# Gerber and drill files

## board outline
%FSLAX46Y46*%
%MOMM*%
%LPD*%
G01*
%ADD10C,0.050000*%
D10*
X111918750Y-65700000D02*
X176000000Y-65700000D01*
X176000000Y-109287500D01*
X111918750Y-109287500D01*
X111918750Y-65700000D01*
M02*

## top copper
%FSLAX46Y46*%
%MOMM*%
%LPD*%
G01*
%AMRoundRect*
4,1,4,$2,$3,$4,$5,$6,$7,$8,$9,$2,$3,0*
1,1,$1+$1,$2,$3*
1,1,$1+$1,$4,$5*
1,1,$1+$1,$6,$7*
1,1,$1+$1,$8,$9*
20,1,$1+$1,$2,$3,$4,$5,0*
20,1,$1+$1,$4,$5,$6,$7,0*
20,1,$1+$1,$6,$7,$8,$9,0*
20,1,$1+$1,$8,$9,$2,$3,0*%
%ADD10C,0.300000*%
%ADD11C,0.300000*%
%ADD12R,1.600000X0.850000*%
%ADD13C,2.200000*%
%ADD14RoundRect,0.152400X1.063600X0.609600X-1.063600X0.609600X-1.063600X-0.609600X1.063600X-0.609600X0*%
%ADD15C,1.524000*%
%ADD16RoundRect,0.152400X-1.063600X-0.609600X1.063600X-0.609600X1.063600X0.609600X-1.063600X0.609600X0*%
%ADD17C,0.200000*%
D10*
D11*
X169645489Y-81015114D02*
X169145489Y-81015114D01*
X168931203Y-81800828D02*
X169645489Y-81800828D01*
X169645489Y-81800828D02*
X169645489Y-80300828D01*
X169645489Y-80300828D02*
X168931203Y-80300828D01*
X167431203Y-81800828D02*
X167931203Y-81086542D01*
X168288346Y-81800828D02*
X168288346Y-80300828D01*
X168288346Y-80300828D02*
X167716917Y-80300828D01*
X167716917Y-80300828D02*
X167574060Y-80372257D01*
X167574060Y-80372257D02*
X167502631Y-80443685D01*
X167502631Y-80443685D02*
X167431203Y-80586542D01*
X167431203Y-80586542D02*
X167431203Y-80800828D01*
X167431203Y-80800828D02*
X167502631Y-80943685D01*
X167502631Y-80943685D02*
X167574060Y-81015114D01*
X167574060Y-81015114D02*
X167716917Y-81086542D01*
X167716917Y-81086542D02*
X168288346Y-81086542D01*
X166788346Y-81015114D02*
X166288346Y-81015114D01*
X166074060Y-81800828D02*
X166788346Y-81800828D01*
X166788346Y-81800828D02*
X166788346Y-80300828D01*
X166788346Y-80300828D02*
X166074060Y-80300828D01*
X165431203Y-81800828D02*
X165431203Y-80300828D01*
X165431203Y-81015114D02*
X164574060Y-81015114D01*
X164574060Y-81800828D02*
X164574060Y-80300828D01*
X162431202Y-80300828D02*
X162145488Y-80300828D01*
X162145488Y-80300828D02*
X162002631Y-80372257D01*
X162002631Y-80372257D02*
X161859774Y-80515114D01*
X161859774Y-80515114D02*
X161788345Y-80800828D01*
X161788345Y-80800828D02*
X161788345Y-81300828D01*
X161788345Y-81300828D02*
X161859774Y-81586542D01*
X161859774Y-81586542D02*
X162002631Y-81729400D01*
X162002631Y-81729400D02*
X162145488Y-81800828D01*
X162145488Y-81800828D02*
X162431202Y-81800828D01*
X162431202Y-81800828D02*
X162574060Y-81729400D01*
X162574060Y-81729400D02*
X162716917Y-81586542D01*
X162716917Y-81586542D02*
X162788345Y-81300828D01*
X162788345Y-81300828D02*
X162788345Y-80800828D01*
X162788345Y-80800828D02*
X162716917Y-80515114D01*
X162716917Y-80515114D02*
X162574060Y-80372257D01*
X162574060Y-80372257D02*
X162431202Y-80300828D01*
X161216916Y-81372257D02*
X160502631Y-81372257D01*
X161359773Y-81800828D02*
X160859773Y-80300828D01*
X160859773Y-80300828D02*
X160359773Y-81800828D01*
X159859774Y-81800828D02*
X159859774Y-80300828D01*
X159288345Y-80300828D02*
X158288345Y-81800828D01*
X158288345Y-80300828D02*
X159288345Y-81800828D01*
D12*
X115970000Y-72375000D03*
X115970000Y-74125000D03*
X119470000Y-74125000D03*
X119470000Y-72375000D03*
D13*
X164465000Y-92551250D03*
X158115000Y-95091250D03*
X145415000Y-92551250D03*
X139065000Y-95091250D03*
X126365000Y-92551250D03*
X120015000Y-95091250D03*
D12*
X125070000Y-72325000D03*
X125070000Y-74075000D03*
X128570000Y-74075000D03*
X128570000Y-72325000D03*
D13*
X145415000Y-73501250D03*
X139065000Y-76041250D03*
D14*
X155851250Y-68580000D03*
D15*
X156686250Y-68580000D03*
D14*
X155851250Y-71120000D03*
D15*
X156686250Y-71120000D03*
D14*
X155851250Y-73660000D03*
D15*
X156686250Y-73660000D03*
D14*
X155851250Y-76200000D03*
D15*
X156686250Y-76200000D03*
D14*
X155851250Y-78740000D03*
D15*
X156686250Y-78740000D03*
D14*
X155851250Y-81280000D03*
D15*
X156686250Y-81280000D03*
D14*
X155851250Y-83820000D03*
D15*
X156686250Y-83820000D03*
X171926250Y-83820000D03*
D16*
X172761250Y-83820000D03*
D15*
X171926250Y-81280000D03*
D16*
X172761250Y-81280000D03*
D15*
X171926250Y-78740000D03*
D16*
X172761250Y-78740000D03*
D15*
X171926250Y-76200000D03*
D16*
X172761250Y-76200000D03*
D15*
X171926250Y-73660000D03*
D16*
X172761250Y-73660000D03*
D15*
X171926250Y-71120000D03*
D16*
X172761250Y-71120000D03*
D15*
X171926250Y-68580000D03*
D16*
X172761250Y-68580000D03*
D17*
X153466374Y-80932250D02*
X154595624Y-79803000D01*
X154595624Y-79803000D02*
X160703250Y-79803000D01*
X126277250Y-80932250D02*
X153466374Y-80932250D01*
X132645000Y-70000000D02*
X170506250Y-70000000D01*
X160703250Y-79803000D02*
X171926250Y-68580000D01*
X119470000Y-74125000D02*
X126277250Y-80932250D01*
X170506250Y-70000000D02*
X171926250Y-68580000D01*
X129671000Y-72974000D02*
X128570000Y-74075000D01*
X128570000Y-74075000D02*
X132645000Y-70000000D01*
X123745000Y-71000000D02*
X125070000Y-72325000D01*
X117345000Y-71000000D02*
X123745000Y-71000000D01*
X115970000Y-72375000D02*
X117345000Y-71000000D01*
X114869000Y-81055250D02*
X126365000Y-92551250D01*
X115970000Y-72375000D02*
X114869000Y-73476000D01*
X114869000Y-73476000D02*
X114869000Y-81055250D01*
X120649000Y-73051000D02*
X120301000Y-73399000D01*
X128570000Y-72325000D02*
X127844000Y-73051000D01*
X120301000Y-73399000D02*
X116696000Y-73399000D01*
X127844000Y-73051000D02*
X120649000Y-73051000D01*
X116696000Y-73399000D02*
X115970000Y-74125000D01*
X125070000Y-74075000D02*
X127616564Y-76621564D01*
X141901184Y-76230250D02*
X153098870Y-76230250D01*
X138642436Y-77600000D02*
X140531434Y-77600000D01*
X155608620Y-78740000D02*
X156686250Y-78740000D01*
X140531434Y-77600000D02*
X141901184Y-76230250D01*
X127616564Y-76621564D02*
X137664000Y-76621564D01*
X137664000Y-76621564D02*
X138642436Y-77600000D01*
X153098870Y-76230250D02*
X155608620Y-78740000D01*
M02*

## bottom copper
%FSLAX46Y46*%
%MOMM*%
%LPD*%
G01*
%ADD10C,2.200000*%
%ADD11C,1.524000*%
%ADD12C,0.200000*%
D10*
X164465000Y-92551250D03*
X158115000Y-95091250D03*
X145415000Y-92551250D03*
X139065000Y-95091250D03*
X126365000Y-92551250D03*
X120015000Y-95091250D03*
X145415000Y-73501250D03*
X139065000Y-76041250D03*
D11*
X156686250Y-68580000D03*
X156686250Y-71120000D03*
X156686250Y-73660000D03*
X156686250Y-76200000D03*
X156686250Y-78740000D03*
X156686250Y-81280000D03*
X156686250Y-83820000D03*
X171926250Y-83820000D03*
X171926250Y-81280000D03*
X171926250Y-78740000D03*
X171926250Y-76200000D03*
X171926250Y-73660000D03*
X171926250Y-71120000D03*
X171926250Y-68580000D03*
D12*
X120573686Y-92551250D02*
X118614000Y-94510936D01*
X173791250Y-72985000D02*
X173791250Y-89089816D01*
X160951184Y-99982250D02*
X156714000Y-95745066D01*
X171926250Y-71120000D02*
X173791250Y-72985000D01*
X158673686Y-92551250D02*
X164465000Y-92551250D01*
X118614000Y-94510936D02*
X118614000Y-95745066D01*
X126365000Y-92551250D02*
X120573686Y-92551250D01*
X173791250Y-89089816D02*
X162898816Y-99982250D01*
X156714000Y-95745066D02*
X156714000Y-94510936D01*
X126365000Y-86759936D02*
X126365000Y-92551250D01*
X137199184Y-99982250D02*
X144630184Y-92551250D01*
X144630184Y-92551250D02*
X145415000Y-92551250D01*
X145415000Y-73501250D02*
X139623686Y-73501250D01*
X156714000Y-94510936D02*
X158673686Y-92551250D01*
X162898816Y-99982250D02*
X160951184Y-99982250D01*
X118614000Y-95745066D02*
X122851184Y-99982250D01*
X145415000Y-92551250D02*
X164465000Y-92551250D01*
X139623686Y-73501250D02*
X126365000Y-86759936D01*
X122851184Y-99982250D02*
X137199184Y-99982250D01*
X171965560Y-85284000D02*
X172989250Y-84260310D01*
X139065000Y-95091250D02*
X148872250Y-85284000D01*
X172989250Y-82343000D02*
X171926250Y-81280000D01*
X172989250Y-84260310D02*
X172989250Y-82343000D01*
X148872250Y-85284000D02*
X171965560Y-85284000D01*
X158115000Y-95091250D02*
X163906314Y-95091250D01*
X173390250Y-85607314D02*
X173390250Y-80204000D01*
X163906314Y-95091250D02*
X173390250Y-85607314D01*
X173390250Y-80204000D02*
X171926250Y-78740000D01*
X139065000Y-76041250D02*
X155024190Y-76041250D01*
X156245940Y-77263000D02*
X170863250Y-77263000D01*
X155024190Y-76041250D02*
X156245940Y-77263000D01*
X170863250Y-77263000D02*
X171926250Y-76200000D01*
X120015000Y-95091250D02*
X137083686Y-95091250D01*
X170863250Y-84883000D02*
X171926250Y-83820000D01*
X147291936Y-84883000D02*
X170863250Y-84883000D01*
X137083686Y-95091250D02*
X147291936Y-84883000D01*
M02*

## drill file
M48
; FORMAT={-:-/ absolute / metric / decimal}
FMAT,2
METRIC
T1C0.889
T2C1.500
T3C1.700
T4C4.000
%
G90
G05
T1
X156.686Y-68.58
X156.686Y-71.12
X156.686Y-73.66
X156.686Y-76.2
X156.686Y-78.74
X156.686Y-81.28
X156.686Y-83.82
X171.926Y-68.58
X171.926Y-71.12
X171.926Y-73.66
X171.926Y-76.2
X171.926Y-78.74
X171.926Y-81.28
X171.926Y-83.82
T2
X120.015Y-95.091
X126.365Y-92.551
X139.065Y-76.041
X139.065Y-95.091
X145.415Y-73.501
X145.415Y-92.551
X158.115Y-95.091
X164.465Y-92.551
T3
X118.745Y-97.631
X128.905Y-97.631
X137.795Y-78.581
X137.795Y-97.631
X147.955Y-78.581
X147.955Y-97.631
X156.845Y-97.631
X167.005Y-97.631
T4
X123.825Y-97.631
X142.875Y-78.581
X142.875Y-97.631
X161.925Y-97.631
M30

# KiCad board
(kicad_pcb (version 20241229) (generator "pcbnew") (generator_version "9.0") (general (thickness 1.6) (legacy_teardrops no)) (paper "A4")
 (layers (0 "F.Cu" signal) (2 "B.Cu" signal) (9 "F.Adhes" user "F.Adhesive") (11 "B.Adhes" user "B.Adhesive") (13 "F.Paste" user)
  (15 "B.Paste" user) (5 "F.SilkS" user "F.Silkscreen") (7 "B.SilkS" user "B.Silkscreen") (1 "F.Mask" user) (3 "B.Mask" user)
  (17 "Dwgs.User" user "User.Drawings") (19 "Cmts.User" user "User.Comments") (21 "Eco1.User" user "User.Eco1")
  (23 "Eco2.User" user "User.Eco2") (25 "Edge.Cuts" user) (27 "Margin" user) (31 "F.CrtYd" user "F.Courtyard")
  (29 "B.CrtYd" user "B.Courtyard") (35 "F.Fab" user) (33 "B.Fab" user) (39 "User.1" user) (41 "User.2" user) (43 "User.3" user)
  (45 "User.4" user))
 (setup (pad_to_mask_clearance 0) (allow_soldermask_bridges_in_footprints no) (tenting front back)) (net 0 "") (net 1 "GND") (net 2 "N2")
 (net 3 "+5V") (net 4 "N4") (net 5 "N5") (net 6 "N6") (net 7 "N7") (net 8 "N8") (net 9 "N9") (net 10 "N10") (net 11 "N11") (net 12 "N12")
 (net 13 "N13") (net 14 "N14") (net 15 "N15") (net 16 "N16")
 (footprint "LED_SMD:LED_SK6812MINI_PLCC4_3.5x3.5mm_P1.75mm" (layer "F.Cu") (at 117.72 73.25)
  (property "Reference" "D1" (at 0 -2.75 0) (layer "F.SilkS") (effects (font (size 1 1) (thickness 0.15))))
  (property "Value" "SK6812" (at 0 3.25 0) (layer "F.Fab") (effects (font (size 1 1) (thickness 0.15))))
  (pad "1" smd rect (at -1.75 -0.875) (size 1.6 0.85) (layers "F.Cu" "F.Mask" "F.Paste") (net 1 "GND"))
  (pad "2" smd rect (at -1.75 0.875) (size 1.6 0.85) (layers "F.Cu" "F.Mask" "F.Paste") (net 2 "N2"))
  (pad "3" smd rect (at 1.75 0.875) (size 1.6 0.85) (layers "F.Cu" "F.Mask" "F.Paste") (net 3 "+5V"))
  (pad "4" smd rect (at 1.75 -0.875) (size 1.6 0.85) (layers "F.Cu" "F.Mask" "F.Paste") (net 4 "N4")))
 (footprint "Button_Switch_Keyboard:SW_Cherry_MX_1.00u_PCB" (layer "F.Cu") (at 164.465 92.55125)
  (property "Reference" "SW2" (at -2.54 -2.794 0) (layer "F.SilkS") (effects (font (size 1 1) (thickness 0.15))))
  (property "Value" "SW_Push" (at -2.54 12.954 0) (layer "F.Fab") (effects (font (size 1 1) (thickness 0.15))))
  (pad "" np_thru_hole circle (at -7.62 5.08) (size 1.7 1.7) (drill 1.7) (layers "*.Cu" "*.Mask"))
  (pad "" np_thru_hole circle (at -2.54 5.08) (size 4 4) (drill 4) (layers "*.Cu" "*.Mask"))
  (pad "" np_thru_hole circle (at 2.54 5.08) (size 1.7 1.7) (drill 1.7) (layers "*.Cu" "*.Mask"))
  (pad "1" thru_hole circle (at 0 0) (size 2.2 2.2) (drill 1.5) (layers "*.Cu" "*.Mask") (remove_unused_layers no) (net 1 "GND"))
  (pad "2" thru_hole circle (at -6.35 2.54) (size 2.2 2.2) (drill 1.5) (layers "*.Cu" "*.Mask") (remove_unused_layers no) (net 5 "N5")))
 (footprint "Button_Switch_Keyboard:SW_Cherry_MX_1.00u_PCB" (layer "F.Cu") (at 145.415 92.55125)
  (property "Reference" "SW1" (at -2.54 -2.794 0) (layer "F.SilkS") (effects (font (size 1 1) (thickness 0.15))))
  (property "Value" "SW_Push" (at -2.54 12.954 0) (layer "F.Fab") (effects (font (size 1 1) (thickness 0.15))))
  (pad "" np_thru_hole circle (at -7.62 5.08) (size 1.7 1.7) (drill 1.7) (layers "*.Cu" "*.Mask"))
  (pad "" np_thru_hole circle (at -2.54 5.08) (size 4 4) (drill 4) (layers "*.Cu" "*.Mask"))
  (pad "" np_thru_hole circle (at 2.54 5.08) (size 1.7 1.7) (drill 1.7) (layers "*.Cu" "*.Mask"))
  (pad "1" thru_hole circle (at 0 0) (size 2.2 2.2) (drill 1.5) (layers "*.Cu" "*.Mask") (remove_unused_layers no) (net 1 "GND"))
  (pad "2" thru_hole circle (at -6.35 2.54) (size 2.2 2.2) (drill 1.5) (layers "*.Cu" "*.Mask") (remove_unused_layers no) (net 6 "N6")))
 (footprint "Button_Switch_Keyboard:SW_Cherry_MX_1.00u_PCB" (layer "F.Cu") (at 126.365 92.55125)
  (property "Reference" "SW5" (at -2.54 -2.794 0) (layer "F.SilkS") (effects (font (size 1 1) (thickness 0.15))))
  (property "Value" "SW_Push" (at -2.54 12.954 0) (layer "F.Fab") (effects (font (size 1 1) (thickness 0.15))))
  (pad "" np_thru_hole circle (at -7.62 5.08) (size 1.7 1.7) (drill 1.7) (layers "*.Cu" "*.Mask"))
  (pad "" np_thru_hole circle (at -2.54 5.08) (size 4 4) (drill 4) (layers "*.Cu" "*.Mask"))
  (pad "" np_thru_hole circle (at 2.54 5.08) (size 1.7 1.7) (drill 1.7) (layers "*.Cu" "*.Mask"))
  (pad "1" thru_hole circle (at 0 0) (size 2.2 2.2) (drill 1.5) (layers "*.Cu" "*.Mask") (remove_unused_layers no) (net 1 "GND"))
  (pad "2" thru_hole circle (at -6.35 2.54) (size 2.2 2.2) (drill 1.5) (layers "*.Cu" "*.Mask") (remove_unused_layers no) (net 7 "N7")))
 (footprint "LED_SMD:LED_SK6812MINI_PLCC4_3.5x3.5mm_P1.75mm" (layer "F.Cu") (at 126.82 73.2)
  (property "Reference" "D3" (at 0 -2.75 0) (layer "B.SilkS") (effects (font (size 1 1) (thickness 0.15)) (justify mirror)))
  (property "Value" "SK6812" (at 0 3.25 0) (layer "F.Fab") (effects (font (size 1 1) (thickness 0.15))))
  (pad "1" smd rect (at -1.75 -0.875) (size 1.6 0.85) (layers "F.Cu" "F.Mask" "F.Paste") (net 1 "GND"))
  (pad "2" smd rect (at -1.75 0.875) (size 1.6 0.85) (layers "F.Cu" "F.Mask" "F.Paste") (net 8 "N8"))
  (pad "3" smd rect (at 1.75 0.875) (size 1.6 0.85) (layers "F.Cu" "F.Mask" "F.Paste") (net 3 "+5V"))
  (pad "4" smd rect (at 1.75 -0.875) (size 1.6 0.85) (layers "F.Cu" "F.Mask" "F.Paste") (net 2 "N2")))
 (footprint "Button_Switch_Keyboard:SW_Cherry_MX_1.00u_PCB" (layer "F.Cu") (at 145.415 73.50125)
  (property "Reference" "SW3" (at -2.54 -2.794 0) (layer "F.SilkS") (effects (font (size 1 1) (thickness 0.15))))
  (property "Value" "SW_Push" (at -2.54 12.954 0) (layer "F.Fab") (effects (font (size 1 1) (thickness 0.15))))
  (pad "" np_thru_hole circle (at -7.62 5.08) (size 1.7 1.7) (drill 1.7) (layers "*.Cu" "*.Mask"))
  (pad "" np_thru_hole circle (at -2.54 5.08) (size 4 4) (drill 4) (layers "*.Cu" "*.Mask"))
  (pad "" np_thru_hole circle (at 2.54 5.08) (size 1.7 1.7) (drill 1.7) (layers "*.Cu" "*.Mask"))
  (pad "1" thru_hole circle (at 0 0) (size 2.2 2.2) (drill 1.5) (layers "*.Cu" "*.Mask") (remove_unused_layers no) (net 1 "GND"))
  (pad "2" thru_hole circle (at -6.35 2.54) (size 2.2 2.2) (drill 1.5) (layers "*.Cu" "*.Mask") (remove_unused_layers no) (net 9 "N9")))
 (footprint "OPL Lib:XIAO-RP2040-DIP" (layer "F.Cu") (at 164.30625 76.2)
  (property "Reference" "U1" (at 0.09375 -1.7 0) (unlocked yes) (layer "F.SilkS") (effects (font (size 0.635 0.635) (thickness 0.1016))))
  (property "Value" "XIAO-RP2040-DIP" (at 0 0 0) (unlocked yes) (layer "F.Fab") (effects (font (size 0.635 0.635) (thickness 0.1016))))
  (pad "1" smd roundrect (at -8.455 -7.62 180) (size 2.432 1.524) (layers "F.Cu" "F.Mask") (roundrect_rratio 0.1) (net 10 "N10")
   (thermal_bridge_angle 45))
  (pad "1" thru_hole circle (at -7.62 -7.62 180) (size 1.524 1.524) (drill 0.889) (layers "*.Cu" "*.Mask") (remove_unused_layers no)
   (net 10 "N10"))
  (pad "2" smd roundrect (at -8.455 -5.08 180) (size 2.432 1.524) (layers "F.Cu" "F.Mask") (roundrect_rratio 0.1) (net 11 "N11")
   (thermal_bridge_angle 45))
  (pad "2" thru_hole circle (at -7.62 -5.08 180) (size 1.524 1.524) (drill 0.889) (layers "*.Cu" "*.Mask") (remove_unused_layers no)
   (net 11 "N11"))
  (pad "3" smd roundrect (at -8.455 -2.54 180) (size 2.432 1.524) (layers "F.Cu" "F.Mask") (roundrect_rratio 0.1) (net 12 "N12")
   (thermal_bridge_angle 45))
  (pad "3" thru_hole circle (at -7.62 -2.54 180) (size 1.524 1.524) (drill 0.889) (layers "*.Cu" "*.Mask") (remove_unused_layers no)
   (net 12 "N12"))
  (pad "4" smd roundrect (at -8.455 0 180) (size 2.432 1.524) (layers "F.Cu" "F.Mask") (roundrect_rratio 0.1) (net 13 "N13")
   (thermal_bridge_angle 45))
  (pad "4" thru_hole circle (at -7.62 0 180) (size 1.524 1.524) (drill 0.889) (layers "*.Cu" "*.Mask") (remove_unused_layers no)
   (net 13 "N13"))
  (pad "5" smd roundrect (at -8.455 2.54 180) (size 2.432 1.524) (layers "F.Cu" "F.Mask") (roundrect_rratio 0.1) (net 8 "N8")
   (thermal_bridge_angle 45))
  (pad "5" thru_hole circle (at -7.62 2.54 180) (size 1.524 1.524) (drill 0.889) (layers "*.Cu" "*.Mask") (remove_unused_layers no)
   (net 8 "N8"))
  (pad "6" smd roundrect (at -8.455 5.08 180) (size 2.432 1.524) (layers "F.Cu" "F.Mask") (roundrect_rratio 0.1) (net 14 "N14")
   (thermal_bridge_angle 45))
  (pad "6" thru_hole circle (at -7.62 5.08 180) (size 1.524 1.524) (drill 0.889) (layers "*.Cu" "*.Mask") (remove_unused_layers no)
   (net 14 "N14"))
  (pad "7" smd roundrect (at -8.455 7.62 180) (size 2.432 1.524) (layers "F.Cu" "F.Mask") (roundrect_rratio 0.1) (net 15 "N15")
   (thermal_bridge_angle 45))
  (pad "7" thru_hole circle (at -7.62 7.62 180) (size 1.524 1.524) (drill 0.889) (layers "*.Cu" "*.Mask") (remove_unused_layers no)
   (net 15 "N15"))
  (pad "8" thru_hole circle (at 7.62 7.62) (size 1.524 1.524) (drill 0.889) (layers "*.Cu" "*.Mask") (remove_unused_layers no) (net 7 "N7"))
  (pad "8" smd roundrect (at 8.455 7.62) (size 2.432 1.524) (layers "F.Cu" "F.Mask") (roundrect_rratio 0.1) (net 7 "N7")
   (thermal_bridge_angle 45))
  (pad "9" thru_hole circle (at 7.62 5.08) (size 1.524 1.524) (drill 0.889) (layers "*.Cu" "*.Mask") (remove_unused_layers no) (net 6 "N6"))
  (pad "9" smd roundrect (at 8.455 5.08) (size 2.432 1.524) (layers "F.Cu" "F.Mask") (roundrect_rratio 0.1) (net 6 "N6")
   (thermal_bridge_angle 45))
  (pad "10" thru_hole circle (at 7.62 2.54) (size 1.524 1.524) (drill 0.889) (layers "*.Cu" "*.Mask") (remove_unused_layers no) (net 5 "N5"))
  (pad "10" smd roundrect (at 8.455 2.54) (size 2.432 1.524) (layers "F.Cu" "F.Mask") (roundrect_rratio 0.1) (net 5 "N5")
   (thermal_bridge_angle 45))
  (pad "11" thru_hole circle (at 7.62 0) (size 1.524 1.524) (drill 0.889) (layers "*.Cu" "*.Mask") (remove_unused_layers no) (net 9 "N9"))
  (pad "11" smd roundrect (at 8.455 0) (size 2.432 1.524) (layers "F.Cu" "F.Mask") (roundrect_rratio 0.1) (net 9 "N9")
   (thermal_bridge_angle 45))
  (pad "12" thru_hole circle (at 7.62 -2.54) (size 1.524 1.524) (drill 0.889) (layers "*.Cu" "*.Mask") (remove_unused_layers no)
   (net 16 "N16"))
  (pad "12" smd roundrect (at 8.455 -2.54) (size 2.432 1.524) (layers "F.Cu" "F.Mask") (roundrect_rratio 0.1) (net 16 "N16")
   (thermal_bridge_angle 45))
  (pad "13" thru_hole circle (at 7.62 -5.08) (size 1.524 1.524) (drill 0.889) (layers "*.Cu" "*.Mask") (remove_unused_layers no)
   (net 1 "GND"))
  (pad "13" smd roundrect (at 8.455 -5.08) (size 2.432 1.524) (layers "F.Cu" "F.Mask") (roundrect_rratio 0.1) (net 1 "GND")
   (thermal_bridge_angle 45))
  (pad "14" thru_hole circle (at 7.62 -7.62) (size 1.524 1.524) (drill 0.889) (layers "*.Cu" "*.Mask") (remove_unused_layers no)
   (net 3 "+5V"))
  (pad "14" smd roundrect (at 8.455 -7.62) (size 2.432 1.524) (layers "F.Cu" "F.Mask") (roundrect_rratio 0.1) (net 3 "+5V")
   (thermal_bridge_angle 45)))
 (gr_rect (start 111.91875 65.7) (end 176 109.2875) (stroke (width 0.05) (type default)) (fill no) (layer "Edge.Cuts"))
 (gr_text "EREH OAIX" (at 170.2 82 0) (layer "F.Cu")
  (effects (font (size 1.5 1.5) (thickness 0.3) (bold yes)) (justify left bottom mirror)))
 (segment (start 153.466374 80.93225) (end 154.595624 79.803) (width 0.2) (layer "F.Cu") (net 3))
 (segment (start 154.595624 79.803) (end 160.70325 79.803) (width 0.2) (layer "F.Cu") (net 3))
 (segment (start 126.27725 80.93225) (end 153.466374 80.93225) (width 0.2) (layer "F.Cu") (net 3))
 (segment (start 132.645 70) (end 170.50625 70) (width 0.2) (layer "F.Cu") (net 3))
 (segment (start 160.70325 79.803) (end 171.92625 68.58) (width 0.2) (layer "F.Cu") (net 3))
 (segment (start 119.47 74.125) (end 126.27725 80.93225) (width 0.2) (layer "F.Cu") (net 3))
 (segment (start 170.50625 70) (end 171.92625 68.58) (width 0.2) (layer "F.Cu") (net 3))
 (segment (start 129.671 72.974) (end 128.57 74.075) (width 0.2) (layer "F.Cu") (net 3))
 (segment (start 128.57 74.075) (end 132.645 70) (width 0.2) (layer "F.Cu") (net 3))
 (segment (start 123.745 71) (end 125.07 72.325) (width 0.2) (layer "F.Cu") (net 1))
 (segment (start 117.345 71) (end 123.745 71) (width 0.2) (layer "F.Cu") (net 1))
 (segment (start 115.97 72.375) (end 117.345 71) (width 0.2) (layer "F.Cu") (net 1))
 (segment (start 114.869 81.05525) (end 126.365 92.55125) (width 0.2) (layer "F.Cu") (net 1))
 (segment (start 115.97 72.375) (end 114.869 73.476) (width 0.2) (layer "F.Cu") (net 1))
 (segment (start 114.869 73.476) (end 114.869 81.05525) (width 0.2) (layer "F.Cu") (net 1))
 (segment (start 120.573686 92.55125) (end 118.614 94.510936) (width 0.2) (layer "B.Cu") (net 1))
 (segment (start 173.79125 72.985) (end 173.79125 89.089816) (width 0.2) (layer "B.Cu") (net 1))
 (segment (start 160.951184 99.98225) (end 156.714 95.745066) (width 0.2) (layer "B.Cu") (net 1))
 (segment (start 171.92625 71.12) (end 173.79125 72.985) (width 0.2) (layer "B.Cu") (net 1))
 (segment (start 158.673686 92.55125) (end 164.465 92.55125) (width 0.2) (layer "B.Cu") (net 1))
 (segment (start 118.614 94.510936) (end 118.614 95.745066) (width 0.2) (layer "B.Cu") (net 1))
 (segment (start 126.365 92.55125) (end 120.573686 92.55125) (width 0.2) (layer "B.Cu") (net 1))
 (segment (start 173.79125 89.089816) (end 162.898816 99.98225) (width 0.2) (layer "B.Cu") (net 1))
 (segment (start 156.714 95.745066) (end 156.714 94.510936) (width 0.2) (layer "B.Cu") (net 1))
 (segment (start 126.365 86.759936) (end 126.365 92.55125) (width 0.2) (layer "B.Cu") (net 1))
 (segment (start 137.199184 99.98225) (end 144.630184 92.55125) (width 0.2) (layer "B.Cu") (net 1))
 (segment (start 144.630184 92.55125) (end 145.415 92.55125) (width 0.2) (layer "B.Cu") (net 1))
 (segment (start 145.415 73.50125) (end 139.623686 73.50125) (width 0.2) (layer "B.Cu") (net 1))
 (segment (start 156.714 94.510936) (end 158.673686 92.55125) (width 0.2) (layer "B.Cu") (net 1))
 (segment (start 162.898816 99.98225) (end 160.951184 99.98225) (width 0.2) (layer "B.Cu") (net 1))
 (segment (start 118.614 95.745066) (end 122.851184 99.98225) (width 0.2) (layer "B.Cu") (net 1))
 (segment (start 145.415 92.55125) (end 164.465 92.55125) (width 0.2) (layer "B.Cu") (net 1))
 (segment (start 139.623686 73.50125) (end 126.365 86.759936) (width 0.2) (layer "B.Cu") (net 1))
 (segment (start 122.851184 99.98225) (end 137.199184 99.98225) (width 0.2) (layer "B.Cu") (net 1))
 (segment (start 120.649 73.051) (end 120.301 73.399) (width 0.2) (layer "F.Cu") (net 2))
 (segment (start 128.57 72.325) (end 127.844 73.051) (width 0.2) (layer "F.Cu") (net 2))
 (segment (start 120.301 73.399) (end 116.696 73.399) (width 0.2) (layer "F.Cu") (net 2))
 (segment (start 127.844 73.051) (end 120.649 73.051) (width 0.2) (layer "F.Cu") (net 2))
 (segment (start 116.696 73.399) (end 115.97 74.125) (width 0.2) (layer "F.Cu") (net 2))
 (segment (start 125.07 74.075) (end 127.616564 76.621564) (width 0.2) (layer "F.Cu") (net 8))
 (segment (start 141.901184 76.23025) (end 153.09887 76.23025) (width 0.2) (layer "F.Cu") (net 8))
 (segment (start 138.642436 77.6) (end 140.531434 77.6) (width 0.2) (layer "F.Cu") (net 8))
 (segment (start 155.60862 78.74) (end 156.68625 78.74) (width 0.2) (layer "F.Cu") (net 8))
 (segment (start 140.531434 77.6) (end 141.901184 76.23025) (width 0.2) (layer "F.Cu") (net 8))
 (segment (start 127.616564 76.621564) (end 137.664 76.621564) (width 0.2) (layer "F.Cu") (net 8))
 (segment (start 137.664 76.621564) (end 138.642436 77.6) (width 0.2) (layer "F.Cu") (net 8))
 (segment (start 153.09887 76.23025) (end 155.60862 78.74) (width 0.2) (layer "F.Cu") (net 8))
 (segment (start 171.96556 85.284) (end 172.98925 84.26031) (width 0.2) (layer "B.Cu") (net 6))
 (segment (start 139.065 95.09125) (end 148.87225 85.284) (width 0.2) (layer "B.Cu") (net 6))
 (segment (start 172.98925 82.343) (end 171.92625 81.28) (width 0.2) (layer "B.Cu") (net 6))
 (segment (start 172.98925 84.26031) (end 172.98925 82.343) (width 0.2) (layer "B.Cu") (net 6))
 (segment (start 148.87225 85.284) (end 171.96556 85.284) (width 0.2) (layer "B.Cu") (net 6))
 (segment (start 158.115 95.09125) (end 163.906314 95.09125) (width 0.2) (layer "B.Cu") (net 5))
 (segment (start 173.39025 85.607314) (end 173.39025 80.204) (width 0.2) (layer "B.Cu") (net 5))
 (segment (start 163.906314 95.09125) (end 173.39025 85.607314) (width 0.2) (layer "B.Cu") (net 5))
 (segment (start 173.39025 80.204) (end 171.92625 78.74) (width 0.2) (layer "B.Cu") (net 5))
 (segment (start 139.065 76.04125) (end 155.02419 76.04125) (width 0.2) (layer "B.Cu") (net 9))
 (segment (start 156.24594 77.263) (end 170.86325 77.263) (width 0.2) (layer "B.Cu") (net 9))
 (segment (start 155.02419 76.04125) (end 156.24594 77.263) (width 0.2) (layer "B.Cu") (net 9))
 (segment (start 170.86325 77.263) (end 171.92625 76.2) (width 0.2) (layer "B.Cu") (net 9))
 (segment (start 120.015 95.09125) (end 137.083686 95.09125) (width 0.2) (layer "B.Cu") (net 7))
 (segment (start 170.86325 84.883) (end 171.92625 83.82) (width 0.2) (layer "B.Cu") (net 7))
 (segment (start 147.291936 84.883) (end 170.86325 84.883) (width 0.2) (layer "B.Cu") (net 7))
 (segment (start 137.083686 95.09125) (end 147.291936 84.883) (width 0.2) (layer "B.Cu") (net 7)))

